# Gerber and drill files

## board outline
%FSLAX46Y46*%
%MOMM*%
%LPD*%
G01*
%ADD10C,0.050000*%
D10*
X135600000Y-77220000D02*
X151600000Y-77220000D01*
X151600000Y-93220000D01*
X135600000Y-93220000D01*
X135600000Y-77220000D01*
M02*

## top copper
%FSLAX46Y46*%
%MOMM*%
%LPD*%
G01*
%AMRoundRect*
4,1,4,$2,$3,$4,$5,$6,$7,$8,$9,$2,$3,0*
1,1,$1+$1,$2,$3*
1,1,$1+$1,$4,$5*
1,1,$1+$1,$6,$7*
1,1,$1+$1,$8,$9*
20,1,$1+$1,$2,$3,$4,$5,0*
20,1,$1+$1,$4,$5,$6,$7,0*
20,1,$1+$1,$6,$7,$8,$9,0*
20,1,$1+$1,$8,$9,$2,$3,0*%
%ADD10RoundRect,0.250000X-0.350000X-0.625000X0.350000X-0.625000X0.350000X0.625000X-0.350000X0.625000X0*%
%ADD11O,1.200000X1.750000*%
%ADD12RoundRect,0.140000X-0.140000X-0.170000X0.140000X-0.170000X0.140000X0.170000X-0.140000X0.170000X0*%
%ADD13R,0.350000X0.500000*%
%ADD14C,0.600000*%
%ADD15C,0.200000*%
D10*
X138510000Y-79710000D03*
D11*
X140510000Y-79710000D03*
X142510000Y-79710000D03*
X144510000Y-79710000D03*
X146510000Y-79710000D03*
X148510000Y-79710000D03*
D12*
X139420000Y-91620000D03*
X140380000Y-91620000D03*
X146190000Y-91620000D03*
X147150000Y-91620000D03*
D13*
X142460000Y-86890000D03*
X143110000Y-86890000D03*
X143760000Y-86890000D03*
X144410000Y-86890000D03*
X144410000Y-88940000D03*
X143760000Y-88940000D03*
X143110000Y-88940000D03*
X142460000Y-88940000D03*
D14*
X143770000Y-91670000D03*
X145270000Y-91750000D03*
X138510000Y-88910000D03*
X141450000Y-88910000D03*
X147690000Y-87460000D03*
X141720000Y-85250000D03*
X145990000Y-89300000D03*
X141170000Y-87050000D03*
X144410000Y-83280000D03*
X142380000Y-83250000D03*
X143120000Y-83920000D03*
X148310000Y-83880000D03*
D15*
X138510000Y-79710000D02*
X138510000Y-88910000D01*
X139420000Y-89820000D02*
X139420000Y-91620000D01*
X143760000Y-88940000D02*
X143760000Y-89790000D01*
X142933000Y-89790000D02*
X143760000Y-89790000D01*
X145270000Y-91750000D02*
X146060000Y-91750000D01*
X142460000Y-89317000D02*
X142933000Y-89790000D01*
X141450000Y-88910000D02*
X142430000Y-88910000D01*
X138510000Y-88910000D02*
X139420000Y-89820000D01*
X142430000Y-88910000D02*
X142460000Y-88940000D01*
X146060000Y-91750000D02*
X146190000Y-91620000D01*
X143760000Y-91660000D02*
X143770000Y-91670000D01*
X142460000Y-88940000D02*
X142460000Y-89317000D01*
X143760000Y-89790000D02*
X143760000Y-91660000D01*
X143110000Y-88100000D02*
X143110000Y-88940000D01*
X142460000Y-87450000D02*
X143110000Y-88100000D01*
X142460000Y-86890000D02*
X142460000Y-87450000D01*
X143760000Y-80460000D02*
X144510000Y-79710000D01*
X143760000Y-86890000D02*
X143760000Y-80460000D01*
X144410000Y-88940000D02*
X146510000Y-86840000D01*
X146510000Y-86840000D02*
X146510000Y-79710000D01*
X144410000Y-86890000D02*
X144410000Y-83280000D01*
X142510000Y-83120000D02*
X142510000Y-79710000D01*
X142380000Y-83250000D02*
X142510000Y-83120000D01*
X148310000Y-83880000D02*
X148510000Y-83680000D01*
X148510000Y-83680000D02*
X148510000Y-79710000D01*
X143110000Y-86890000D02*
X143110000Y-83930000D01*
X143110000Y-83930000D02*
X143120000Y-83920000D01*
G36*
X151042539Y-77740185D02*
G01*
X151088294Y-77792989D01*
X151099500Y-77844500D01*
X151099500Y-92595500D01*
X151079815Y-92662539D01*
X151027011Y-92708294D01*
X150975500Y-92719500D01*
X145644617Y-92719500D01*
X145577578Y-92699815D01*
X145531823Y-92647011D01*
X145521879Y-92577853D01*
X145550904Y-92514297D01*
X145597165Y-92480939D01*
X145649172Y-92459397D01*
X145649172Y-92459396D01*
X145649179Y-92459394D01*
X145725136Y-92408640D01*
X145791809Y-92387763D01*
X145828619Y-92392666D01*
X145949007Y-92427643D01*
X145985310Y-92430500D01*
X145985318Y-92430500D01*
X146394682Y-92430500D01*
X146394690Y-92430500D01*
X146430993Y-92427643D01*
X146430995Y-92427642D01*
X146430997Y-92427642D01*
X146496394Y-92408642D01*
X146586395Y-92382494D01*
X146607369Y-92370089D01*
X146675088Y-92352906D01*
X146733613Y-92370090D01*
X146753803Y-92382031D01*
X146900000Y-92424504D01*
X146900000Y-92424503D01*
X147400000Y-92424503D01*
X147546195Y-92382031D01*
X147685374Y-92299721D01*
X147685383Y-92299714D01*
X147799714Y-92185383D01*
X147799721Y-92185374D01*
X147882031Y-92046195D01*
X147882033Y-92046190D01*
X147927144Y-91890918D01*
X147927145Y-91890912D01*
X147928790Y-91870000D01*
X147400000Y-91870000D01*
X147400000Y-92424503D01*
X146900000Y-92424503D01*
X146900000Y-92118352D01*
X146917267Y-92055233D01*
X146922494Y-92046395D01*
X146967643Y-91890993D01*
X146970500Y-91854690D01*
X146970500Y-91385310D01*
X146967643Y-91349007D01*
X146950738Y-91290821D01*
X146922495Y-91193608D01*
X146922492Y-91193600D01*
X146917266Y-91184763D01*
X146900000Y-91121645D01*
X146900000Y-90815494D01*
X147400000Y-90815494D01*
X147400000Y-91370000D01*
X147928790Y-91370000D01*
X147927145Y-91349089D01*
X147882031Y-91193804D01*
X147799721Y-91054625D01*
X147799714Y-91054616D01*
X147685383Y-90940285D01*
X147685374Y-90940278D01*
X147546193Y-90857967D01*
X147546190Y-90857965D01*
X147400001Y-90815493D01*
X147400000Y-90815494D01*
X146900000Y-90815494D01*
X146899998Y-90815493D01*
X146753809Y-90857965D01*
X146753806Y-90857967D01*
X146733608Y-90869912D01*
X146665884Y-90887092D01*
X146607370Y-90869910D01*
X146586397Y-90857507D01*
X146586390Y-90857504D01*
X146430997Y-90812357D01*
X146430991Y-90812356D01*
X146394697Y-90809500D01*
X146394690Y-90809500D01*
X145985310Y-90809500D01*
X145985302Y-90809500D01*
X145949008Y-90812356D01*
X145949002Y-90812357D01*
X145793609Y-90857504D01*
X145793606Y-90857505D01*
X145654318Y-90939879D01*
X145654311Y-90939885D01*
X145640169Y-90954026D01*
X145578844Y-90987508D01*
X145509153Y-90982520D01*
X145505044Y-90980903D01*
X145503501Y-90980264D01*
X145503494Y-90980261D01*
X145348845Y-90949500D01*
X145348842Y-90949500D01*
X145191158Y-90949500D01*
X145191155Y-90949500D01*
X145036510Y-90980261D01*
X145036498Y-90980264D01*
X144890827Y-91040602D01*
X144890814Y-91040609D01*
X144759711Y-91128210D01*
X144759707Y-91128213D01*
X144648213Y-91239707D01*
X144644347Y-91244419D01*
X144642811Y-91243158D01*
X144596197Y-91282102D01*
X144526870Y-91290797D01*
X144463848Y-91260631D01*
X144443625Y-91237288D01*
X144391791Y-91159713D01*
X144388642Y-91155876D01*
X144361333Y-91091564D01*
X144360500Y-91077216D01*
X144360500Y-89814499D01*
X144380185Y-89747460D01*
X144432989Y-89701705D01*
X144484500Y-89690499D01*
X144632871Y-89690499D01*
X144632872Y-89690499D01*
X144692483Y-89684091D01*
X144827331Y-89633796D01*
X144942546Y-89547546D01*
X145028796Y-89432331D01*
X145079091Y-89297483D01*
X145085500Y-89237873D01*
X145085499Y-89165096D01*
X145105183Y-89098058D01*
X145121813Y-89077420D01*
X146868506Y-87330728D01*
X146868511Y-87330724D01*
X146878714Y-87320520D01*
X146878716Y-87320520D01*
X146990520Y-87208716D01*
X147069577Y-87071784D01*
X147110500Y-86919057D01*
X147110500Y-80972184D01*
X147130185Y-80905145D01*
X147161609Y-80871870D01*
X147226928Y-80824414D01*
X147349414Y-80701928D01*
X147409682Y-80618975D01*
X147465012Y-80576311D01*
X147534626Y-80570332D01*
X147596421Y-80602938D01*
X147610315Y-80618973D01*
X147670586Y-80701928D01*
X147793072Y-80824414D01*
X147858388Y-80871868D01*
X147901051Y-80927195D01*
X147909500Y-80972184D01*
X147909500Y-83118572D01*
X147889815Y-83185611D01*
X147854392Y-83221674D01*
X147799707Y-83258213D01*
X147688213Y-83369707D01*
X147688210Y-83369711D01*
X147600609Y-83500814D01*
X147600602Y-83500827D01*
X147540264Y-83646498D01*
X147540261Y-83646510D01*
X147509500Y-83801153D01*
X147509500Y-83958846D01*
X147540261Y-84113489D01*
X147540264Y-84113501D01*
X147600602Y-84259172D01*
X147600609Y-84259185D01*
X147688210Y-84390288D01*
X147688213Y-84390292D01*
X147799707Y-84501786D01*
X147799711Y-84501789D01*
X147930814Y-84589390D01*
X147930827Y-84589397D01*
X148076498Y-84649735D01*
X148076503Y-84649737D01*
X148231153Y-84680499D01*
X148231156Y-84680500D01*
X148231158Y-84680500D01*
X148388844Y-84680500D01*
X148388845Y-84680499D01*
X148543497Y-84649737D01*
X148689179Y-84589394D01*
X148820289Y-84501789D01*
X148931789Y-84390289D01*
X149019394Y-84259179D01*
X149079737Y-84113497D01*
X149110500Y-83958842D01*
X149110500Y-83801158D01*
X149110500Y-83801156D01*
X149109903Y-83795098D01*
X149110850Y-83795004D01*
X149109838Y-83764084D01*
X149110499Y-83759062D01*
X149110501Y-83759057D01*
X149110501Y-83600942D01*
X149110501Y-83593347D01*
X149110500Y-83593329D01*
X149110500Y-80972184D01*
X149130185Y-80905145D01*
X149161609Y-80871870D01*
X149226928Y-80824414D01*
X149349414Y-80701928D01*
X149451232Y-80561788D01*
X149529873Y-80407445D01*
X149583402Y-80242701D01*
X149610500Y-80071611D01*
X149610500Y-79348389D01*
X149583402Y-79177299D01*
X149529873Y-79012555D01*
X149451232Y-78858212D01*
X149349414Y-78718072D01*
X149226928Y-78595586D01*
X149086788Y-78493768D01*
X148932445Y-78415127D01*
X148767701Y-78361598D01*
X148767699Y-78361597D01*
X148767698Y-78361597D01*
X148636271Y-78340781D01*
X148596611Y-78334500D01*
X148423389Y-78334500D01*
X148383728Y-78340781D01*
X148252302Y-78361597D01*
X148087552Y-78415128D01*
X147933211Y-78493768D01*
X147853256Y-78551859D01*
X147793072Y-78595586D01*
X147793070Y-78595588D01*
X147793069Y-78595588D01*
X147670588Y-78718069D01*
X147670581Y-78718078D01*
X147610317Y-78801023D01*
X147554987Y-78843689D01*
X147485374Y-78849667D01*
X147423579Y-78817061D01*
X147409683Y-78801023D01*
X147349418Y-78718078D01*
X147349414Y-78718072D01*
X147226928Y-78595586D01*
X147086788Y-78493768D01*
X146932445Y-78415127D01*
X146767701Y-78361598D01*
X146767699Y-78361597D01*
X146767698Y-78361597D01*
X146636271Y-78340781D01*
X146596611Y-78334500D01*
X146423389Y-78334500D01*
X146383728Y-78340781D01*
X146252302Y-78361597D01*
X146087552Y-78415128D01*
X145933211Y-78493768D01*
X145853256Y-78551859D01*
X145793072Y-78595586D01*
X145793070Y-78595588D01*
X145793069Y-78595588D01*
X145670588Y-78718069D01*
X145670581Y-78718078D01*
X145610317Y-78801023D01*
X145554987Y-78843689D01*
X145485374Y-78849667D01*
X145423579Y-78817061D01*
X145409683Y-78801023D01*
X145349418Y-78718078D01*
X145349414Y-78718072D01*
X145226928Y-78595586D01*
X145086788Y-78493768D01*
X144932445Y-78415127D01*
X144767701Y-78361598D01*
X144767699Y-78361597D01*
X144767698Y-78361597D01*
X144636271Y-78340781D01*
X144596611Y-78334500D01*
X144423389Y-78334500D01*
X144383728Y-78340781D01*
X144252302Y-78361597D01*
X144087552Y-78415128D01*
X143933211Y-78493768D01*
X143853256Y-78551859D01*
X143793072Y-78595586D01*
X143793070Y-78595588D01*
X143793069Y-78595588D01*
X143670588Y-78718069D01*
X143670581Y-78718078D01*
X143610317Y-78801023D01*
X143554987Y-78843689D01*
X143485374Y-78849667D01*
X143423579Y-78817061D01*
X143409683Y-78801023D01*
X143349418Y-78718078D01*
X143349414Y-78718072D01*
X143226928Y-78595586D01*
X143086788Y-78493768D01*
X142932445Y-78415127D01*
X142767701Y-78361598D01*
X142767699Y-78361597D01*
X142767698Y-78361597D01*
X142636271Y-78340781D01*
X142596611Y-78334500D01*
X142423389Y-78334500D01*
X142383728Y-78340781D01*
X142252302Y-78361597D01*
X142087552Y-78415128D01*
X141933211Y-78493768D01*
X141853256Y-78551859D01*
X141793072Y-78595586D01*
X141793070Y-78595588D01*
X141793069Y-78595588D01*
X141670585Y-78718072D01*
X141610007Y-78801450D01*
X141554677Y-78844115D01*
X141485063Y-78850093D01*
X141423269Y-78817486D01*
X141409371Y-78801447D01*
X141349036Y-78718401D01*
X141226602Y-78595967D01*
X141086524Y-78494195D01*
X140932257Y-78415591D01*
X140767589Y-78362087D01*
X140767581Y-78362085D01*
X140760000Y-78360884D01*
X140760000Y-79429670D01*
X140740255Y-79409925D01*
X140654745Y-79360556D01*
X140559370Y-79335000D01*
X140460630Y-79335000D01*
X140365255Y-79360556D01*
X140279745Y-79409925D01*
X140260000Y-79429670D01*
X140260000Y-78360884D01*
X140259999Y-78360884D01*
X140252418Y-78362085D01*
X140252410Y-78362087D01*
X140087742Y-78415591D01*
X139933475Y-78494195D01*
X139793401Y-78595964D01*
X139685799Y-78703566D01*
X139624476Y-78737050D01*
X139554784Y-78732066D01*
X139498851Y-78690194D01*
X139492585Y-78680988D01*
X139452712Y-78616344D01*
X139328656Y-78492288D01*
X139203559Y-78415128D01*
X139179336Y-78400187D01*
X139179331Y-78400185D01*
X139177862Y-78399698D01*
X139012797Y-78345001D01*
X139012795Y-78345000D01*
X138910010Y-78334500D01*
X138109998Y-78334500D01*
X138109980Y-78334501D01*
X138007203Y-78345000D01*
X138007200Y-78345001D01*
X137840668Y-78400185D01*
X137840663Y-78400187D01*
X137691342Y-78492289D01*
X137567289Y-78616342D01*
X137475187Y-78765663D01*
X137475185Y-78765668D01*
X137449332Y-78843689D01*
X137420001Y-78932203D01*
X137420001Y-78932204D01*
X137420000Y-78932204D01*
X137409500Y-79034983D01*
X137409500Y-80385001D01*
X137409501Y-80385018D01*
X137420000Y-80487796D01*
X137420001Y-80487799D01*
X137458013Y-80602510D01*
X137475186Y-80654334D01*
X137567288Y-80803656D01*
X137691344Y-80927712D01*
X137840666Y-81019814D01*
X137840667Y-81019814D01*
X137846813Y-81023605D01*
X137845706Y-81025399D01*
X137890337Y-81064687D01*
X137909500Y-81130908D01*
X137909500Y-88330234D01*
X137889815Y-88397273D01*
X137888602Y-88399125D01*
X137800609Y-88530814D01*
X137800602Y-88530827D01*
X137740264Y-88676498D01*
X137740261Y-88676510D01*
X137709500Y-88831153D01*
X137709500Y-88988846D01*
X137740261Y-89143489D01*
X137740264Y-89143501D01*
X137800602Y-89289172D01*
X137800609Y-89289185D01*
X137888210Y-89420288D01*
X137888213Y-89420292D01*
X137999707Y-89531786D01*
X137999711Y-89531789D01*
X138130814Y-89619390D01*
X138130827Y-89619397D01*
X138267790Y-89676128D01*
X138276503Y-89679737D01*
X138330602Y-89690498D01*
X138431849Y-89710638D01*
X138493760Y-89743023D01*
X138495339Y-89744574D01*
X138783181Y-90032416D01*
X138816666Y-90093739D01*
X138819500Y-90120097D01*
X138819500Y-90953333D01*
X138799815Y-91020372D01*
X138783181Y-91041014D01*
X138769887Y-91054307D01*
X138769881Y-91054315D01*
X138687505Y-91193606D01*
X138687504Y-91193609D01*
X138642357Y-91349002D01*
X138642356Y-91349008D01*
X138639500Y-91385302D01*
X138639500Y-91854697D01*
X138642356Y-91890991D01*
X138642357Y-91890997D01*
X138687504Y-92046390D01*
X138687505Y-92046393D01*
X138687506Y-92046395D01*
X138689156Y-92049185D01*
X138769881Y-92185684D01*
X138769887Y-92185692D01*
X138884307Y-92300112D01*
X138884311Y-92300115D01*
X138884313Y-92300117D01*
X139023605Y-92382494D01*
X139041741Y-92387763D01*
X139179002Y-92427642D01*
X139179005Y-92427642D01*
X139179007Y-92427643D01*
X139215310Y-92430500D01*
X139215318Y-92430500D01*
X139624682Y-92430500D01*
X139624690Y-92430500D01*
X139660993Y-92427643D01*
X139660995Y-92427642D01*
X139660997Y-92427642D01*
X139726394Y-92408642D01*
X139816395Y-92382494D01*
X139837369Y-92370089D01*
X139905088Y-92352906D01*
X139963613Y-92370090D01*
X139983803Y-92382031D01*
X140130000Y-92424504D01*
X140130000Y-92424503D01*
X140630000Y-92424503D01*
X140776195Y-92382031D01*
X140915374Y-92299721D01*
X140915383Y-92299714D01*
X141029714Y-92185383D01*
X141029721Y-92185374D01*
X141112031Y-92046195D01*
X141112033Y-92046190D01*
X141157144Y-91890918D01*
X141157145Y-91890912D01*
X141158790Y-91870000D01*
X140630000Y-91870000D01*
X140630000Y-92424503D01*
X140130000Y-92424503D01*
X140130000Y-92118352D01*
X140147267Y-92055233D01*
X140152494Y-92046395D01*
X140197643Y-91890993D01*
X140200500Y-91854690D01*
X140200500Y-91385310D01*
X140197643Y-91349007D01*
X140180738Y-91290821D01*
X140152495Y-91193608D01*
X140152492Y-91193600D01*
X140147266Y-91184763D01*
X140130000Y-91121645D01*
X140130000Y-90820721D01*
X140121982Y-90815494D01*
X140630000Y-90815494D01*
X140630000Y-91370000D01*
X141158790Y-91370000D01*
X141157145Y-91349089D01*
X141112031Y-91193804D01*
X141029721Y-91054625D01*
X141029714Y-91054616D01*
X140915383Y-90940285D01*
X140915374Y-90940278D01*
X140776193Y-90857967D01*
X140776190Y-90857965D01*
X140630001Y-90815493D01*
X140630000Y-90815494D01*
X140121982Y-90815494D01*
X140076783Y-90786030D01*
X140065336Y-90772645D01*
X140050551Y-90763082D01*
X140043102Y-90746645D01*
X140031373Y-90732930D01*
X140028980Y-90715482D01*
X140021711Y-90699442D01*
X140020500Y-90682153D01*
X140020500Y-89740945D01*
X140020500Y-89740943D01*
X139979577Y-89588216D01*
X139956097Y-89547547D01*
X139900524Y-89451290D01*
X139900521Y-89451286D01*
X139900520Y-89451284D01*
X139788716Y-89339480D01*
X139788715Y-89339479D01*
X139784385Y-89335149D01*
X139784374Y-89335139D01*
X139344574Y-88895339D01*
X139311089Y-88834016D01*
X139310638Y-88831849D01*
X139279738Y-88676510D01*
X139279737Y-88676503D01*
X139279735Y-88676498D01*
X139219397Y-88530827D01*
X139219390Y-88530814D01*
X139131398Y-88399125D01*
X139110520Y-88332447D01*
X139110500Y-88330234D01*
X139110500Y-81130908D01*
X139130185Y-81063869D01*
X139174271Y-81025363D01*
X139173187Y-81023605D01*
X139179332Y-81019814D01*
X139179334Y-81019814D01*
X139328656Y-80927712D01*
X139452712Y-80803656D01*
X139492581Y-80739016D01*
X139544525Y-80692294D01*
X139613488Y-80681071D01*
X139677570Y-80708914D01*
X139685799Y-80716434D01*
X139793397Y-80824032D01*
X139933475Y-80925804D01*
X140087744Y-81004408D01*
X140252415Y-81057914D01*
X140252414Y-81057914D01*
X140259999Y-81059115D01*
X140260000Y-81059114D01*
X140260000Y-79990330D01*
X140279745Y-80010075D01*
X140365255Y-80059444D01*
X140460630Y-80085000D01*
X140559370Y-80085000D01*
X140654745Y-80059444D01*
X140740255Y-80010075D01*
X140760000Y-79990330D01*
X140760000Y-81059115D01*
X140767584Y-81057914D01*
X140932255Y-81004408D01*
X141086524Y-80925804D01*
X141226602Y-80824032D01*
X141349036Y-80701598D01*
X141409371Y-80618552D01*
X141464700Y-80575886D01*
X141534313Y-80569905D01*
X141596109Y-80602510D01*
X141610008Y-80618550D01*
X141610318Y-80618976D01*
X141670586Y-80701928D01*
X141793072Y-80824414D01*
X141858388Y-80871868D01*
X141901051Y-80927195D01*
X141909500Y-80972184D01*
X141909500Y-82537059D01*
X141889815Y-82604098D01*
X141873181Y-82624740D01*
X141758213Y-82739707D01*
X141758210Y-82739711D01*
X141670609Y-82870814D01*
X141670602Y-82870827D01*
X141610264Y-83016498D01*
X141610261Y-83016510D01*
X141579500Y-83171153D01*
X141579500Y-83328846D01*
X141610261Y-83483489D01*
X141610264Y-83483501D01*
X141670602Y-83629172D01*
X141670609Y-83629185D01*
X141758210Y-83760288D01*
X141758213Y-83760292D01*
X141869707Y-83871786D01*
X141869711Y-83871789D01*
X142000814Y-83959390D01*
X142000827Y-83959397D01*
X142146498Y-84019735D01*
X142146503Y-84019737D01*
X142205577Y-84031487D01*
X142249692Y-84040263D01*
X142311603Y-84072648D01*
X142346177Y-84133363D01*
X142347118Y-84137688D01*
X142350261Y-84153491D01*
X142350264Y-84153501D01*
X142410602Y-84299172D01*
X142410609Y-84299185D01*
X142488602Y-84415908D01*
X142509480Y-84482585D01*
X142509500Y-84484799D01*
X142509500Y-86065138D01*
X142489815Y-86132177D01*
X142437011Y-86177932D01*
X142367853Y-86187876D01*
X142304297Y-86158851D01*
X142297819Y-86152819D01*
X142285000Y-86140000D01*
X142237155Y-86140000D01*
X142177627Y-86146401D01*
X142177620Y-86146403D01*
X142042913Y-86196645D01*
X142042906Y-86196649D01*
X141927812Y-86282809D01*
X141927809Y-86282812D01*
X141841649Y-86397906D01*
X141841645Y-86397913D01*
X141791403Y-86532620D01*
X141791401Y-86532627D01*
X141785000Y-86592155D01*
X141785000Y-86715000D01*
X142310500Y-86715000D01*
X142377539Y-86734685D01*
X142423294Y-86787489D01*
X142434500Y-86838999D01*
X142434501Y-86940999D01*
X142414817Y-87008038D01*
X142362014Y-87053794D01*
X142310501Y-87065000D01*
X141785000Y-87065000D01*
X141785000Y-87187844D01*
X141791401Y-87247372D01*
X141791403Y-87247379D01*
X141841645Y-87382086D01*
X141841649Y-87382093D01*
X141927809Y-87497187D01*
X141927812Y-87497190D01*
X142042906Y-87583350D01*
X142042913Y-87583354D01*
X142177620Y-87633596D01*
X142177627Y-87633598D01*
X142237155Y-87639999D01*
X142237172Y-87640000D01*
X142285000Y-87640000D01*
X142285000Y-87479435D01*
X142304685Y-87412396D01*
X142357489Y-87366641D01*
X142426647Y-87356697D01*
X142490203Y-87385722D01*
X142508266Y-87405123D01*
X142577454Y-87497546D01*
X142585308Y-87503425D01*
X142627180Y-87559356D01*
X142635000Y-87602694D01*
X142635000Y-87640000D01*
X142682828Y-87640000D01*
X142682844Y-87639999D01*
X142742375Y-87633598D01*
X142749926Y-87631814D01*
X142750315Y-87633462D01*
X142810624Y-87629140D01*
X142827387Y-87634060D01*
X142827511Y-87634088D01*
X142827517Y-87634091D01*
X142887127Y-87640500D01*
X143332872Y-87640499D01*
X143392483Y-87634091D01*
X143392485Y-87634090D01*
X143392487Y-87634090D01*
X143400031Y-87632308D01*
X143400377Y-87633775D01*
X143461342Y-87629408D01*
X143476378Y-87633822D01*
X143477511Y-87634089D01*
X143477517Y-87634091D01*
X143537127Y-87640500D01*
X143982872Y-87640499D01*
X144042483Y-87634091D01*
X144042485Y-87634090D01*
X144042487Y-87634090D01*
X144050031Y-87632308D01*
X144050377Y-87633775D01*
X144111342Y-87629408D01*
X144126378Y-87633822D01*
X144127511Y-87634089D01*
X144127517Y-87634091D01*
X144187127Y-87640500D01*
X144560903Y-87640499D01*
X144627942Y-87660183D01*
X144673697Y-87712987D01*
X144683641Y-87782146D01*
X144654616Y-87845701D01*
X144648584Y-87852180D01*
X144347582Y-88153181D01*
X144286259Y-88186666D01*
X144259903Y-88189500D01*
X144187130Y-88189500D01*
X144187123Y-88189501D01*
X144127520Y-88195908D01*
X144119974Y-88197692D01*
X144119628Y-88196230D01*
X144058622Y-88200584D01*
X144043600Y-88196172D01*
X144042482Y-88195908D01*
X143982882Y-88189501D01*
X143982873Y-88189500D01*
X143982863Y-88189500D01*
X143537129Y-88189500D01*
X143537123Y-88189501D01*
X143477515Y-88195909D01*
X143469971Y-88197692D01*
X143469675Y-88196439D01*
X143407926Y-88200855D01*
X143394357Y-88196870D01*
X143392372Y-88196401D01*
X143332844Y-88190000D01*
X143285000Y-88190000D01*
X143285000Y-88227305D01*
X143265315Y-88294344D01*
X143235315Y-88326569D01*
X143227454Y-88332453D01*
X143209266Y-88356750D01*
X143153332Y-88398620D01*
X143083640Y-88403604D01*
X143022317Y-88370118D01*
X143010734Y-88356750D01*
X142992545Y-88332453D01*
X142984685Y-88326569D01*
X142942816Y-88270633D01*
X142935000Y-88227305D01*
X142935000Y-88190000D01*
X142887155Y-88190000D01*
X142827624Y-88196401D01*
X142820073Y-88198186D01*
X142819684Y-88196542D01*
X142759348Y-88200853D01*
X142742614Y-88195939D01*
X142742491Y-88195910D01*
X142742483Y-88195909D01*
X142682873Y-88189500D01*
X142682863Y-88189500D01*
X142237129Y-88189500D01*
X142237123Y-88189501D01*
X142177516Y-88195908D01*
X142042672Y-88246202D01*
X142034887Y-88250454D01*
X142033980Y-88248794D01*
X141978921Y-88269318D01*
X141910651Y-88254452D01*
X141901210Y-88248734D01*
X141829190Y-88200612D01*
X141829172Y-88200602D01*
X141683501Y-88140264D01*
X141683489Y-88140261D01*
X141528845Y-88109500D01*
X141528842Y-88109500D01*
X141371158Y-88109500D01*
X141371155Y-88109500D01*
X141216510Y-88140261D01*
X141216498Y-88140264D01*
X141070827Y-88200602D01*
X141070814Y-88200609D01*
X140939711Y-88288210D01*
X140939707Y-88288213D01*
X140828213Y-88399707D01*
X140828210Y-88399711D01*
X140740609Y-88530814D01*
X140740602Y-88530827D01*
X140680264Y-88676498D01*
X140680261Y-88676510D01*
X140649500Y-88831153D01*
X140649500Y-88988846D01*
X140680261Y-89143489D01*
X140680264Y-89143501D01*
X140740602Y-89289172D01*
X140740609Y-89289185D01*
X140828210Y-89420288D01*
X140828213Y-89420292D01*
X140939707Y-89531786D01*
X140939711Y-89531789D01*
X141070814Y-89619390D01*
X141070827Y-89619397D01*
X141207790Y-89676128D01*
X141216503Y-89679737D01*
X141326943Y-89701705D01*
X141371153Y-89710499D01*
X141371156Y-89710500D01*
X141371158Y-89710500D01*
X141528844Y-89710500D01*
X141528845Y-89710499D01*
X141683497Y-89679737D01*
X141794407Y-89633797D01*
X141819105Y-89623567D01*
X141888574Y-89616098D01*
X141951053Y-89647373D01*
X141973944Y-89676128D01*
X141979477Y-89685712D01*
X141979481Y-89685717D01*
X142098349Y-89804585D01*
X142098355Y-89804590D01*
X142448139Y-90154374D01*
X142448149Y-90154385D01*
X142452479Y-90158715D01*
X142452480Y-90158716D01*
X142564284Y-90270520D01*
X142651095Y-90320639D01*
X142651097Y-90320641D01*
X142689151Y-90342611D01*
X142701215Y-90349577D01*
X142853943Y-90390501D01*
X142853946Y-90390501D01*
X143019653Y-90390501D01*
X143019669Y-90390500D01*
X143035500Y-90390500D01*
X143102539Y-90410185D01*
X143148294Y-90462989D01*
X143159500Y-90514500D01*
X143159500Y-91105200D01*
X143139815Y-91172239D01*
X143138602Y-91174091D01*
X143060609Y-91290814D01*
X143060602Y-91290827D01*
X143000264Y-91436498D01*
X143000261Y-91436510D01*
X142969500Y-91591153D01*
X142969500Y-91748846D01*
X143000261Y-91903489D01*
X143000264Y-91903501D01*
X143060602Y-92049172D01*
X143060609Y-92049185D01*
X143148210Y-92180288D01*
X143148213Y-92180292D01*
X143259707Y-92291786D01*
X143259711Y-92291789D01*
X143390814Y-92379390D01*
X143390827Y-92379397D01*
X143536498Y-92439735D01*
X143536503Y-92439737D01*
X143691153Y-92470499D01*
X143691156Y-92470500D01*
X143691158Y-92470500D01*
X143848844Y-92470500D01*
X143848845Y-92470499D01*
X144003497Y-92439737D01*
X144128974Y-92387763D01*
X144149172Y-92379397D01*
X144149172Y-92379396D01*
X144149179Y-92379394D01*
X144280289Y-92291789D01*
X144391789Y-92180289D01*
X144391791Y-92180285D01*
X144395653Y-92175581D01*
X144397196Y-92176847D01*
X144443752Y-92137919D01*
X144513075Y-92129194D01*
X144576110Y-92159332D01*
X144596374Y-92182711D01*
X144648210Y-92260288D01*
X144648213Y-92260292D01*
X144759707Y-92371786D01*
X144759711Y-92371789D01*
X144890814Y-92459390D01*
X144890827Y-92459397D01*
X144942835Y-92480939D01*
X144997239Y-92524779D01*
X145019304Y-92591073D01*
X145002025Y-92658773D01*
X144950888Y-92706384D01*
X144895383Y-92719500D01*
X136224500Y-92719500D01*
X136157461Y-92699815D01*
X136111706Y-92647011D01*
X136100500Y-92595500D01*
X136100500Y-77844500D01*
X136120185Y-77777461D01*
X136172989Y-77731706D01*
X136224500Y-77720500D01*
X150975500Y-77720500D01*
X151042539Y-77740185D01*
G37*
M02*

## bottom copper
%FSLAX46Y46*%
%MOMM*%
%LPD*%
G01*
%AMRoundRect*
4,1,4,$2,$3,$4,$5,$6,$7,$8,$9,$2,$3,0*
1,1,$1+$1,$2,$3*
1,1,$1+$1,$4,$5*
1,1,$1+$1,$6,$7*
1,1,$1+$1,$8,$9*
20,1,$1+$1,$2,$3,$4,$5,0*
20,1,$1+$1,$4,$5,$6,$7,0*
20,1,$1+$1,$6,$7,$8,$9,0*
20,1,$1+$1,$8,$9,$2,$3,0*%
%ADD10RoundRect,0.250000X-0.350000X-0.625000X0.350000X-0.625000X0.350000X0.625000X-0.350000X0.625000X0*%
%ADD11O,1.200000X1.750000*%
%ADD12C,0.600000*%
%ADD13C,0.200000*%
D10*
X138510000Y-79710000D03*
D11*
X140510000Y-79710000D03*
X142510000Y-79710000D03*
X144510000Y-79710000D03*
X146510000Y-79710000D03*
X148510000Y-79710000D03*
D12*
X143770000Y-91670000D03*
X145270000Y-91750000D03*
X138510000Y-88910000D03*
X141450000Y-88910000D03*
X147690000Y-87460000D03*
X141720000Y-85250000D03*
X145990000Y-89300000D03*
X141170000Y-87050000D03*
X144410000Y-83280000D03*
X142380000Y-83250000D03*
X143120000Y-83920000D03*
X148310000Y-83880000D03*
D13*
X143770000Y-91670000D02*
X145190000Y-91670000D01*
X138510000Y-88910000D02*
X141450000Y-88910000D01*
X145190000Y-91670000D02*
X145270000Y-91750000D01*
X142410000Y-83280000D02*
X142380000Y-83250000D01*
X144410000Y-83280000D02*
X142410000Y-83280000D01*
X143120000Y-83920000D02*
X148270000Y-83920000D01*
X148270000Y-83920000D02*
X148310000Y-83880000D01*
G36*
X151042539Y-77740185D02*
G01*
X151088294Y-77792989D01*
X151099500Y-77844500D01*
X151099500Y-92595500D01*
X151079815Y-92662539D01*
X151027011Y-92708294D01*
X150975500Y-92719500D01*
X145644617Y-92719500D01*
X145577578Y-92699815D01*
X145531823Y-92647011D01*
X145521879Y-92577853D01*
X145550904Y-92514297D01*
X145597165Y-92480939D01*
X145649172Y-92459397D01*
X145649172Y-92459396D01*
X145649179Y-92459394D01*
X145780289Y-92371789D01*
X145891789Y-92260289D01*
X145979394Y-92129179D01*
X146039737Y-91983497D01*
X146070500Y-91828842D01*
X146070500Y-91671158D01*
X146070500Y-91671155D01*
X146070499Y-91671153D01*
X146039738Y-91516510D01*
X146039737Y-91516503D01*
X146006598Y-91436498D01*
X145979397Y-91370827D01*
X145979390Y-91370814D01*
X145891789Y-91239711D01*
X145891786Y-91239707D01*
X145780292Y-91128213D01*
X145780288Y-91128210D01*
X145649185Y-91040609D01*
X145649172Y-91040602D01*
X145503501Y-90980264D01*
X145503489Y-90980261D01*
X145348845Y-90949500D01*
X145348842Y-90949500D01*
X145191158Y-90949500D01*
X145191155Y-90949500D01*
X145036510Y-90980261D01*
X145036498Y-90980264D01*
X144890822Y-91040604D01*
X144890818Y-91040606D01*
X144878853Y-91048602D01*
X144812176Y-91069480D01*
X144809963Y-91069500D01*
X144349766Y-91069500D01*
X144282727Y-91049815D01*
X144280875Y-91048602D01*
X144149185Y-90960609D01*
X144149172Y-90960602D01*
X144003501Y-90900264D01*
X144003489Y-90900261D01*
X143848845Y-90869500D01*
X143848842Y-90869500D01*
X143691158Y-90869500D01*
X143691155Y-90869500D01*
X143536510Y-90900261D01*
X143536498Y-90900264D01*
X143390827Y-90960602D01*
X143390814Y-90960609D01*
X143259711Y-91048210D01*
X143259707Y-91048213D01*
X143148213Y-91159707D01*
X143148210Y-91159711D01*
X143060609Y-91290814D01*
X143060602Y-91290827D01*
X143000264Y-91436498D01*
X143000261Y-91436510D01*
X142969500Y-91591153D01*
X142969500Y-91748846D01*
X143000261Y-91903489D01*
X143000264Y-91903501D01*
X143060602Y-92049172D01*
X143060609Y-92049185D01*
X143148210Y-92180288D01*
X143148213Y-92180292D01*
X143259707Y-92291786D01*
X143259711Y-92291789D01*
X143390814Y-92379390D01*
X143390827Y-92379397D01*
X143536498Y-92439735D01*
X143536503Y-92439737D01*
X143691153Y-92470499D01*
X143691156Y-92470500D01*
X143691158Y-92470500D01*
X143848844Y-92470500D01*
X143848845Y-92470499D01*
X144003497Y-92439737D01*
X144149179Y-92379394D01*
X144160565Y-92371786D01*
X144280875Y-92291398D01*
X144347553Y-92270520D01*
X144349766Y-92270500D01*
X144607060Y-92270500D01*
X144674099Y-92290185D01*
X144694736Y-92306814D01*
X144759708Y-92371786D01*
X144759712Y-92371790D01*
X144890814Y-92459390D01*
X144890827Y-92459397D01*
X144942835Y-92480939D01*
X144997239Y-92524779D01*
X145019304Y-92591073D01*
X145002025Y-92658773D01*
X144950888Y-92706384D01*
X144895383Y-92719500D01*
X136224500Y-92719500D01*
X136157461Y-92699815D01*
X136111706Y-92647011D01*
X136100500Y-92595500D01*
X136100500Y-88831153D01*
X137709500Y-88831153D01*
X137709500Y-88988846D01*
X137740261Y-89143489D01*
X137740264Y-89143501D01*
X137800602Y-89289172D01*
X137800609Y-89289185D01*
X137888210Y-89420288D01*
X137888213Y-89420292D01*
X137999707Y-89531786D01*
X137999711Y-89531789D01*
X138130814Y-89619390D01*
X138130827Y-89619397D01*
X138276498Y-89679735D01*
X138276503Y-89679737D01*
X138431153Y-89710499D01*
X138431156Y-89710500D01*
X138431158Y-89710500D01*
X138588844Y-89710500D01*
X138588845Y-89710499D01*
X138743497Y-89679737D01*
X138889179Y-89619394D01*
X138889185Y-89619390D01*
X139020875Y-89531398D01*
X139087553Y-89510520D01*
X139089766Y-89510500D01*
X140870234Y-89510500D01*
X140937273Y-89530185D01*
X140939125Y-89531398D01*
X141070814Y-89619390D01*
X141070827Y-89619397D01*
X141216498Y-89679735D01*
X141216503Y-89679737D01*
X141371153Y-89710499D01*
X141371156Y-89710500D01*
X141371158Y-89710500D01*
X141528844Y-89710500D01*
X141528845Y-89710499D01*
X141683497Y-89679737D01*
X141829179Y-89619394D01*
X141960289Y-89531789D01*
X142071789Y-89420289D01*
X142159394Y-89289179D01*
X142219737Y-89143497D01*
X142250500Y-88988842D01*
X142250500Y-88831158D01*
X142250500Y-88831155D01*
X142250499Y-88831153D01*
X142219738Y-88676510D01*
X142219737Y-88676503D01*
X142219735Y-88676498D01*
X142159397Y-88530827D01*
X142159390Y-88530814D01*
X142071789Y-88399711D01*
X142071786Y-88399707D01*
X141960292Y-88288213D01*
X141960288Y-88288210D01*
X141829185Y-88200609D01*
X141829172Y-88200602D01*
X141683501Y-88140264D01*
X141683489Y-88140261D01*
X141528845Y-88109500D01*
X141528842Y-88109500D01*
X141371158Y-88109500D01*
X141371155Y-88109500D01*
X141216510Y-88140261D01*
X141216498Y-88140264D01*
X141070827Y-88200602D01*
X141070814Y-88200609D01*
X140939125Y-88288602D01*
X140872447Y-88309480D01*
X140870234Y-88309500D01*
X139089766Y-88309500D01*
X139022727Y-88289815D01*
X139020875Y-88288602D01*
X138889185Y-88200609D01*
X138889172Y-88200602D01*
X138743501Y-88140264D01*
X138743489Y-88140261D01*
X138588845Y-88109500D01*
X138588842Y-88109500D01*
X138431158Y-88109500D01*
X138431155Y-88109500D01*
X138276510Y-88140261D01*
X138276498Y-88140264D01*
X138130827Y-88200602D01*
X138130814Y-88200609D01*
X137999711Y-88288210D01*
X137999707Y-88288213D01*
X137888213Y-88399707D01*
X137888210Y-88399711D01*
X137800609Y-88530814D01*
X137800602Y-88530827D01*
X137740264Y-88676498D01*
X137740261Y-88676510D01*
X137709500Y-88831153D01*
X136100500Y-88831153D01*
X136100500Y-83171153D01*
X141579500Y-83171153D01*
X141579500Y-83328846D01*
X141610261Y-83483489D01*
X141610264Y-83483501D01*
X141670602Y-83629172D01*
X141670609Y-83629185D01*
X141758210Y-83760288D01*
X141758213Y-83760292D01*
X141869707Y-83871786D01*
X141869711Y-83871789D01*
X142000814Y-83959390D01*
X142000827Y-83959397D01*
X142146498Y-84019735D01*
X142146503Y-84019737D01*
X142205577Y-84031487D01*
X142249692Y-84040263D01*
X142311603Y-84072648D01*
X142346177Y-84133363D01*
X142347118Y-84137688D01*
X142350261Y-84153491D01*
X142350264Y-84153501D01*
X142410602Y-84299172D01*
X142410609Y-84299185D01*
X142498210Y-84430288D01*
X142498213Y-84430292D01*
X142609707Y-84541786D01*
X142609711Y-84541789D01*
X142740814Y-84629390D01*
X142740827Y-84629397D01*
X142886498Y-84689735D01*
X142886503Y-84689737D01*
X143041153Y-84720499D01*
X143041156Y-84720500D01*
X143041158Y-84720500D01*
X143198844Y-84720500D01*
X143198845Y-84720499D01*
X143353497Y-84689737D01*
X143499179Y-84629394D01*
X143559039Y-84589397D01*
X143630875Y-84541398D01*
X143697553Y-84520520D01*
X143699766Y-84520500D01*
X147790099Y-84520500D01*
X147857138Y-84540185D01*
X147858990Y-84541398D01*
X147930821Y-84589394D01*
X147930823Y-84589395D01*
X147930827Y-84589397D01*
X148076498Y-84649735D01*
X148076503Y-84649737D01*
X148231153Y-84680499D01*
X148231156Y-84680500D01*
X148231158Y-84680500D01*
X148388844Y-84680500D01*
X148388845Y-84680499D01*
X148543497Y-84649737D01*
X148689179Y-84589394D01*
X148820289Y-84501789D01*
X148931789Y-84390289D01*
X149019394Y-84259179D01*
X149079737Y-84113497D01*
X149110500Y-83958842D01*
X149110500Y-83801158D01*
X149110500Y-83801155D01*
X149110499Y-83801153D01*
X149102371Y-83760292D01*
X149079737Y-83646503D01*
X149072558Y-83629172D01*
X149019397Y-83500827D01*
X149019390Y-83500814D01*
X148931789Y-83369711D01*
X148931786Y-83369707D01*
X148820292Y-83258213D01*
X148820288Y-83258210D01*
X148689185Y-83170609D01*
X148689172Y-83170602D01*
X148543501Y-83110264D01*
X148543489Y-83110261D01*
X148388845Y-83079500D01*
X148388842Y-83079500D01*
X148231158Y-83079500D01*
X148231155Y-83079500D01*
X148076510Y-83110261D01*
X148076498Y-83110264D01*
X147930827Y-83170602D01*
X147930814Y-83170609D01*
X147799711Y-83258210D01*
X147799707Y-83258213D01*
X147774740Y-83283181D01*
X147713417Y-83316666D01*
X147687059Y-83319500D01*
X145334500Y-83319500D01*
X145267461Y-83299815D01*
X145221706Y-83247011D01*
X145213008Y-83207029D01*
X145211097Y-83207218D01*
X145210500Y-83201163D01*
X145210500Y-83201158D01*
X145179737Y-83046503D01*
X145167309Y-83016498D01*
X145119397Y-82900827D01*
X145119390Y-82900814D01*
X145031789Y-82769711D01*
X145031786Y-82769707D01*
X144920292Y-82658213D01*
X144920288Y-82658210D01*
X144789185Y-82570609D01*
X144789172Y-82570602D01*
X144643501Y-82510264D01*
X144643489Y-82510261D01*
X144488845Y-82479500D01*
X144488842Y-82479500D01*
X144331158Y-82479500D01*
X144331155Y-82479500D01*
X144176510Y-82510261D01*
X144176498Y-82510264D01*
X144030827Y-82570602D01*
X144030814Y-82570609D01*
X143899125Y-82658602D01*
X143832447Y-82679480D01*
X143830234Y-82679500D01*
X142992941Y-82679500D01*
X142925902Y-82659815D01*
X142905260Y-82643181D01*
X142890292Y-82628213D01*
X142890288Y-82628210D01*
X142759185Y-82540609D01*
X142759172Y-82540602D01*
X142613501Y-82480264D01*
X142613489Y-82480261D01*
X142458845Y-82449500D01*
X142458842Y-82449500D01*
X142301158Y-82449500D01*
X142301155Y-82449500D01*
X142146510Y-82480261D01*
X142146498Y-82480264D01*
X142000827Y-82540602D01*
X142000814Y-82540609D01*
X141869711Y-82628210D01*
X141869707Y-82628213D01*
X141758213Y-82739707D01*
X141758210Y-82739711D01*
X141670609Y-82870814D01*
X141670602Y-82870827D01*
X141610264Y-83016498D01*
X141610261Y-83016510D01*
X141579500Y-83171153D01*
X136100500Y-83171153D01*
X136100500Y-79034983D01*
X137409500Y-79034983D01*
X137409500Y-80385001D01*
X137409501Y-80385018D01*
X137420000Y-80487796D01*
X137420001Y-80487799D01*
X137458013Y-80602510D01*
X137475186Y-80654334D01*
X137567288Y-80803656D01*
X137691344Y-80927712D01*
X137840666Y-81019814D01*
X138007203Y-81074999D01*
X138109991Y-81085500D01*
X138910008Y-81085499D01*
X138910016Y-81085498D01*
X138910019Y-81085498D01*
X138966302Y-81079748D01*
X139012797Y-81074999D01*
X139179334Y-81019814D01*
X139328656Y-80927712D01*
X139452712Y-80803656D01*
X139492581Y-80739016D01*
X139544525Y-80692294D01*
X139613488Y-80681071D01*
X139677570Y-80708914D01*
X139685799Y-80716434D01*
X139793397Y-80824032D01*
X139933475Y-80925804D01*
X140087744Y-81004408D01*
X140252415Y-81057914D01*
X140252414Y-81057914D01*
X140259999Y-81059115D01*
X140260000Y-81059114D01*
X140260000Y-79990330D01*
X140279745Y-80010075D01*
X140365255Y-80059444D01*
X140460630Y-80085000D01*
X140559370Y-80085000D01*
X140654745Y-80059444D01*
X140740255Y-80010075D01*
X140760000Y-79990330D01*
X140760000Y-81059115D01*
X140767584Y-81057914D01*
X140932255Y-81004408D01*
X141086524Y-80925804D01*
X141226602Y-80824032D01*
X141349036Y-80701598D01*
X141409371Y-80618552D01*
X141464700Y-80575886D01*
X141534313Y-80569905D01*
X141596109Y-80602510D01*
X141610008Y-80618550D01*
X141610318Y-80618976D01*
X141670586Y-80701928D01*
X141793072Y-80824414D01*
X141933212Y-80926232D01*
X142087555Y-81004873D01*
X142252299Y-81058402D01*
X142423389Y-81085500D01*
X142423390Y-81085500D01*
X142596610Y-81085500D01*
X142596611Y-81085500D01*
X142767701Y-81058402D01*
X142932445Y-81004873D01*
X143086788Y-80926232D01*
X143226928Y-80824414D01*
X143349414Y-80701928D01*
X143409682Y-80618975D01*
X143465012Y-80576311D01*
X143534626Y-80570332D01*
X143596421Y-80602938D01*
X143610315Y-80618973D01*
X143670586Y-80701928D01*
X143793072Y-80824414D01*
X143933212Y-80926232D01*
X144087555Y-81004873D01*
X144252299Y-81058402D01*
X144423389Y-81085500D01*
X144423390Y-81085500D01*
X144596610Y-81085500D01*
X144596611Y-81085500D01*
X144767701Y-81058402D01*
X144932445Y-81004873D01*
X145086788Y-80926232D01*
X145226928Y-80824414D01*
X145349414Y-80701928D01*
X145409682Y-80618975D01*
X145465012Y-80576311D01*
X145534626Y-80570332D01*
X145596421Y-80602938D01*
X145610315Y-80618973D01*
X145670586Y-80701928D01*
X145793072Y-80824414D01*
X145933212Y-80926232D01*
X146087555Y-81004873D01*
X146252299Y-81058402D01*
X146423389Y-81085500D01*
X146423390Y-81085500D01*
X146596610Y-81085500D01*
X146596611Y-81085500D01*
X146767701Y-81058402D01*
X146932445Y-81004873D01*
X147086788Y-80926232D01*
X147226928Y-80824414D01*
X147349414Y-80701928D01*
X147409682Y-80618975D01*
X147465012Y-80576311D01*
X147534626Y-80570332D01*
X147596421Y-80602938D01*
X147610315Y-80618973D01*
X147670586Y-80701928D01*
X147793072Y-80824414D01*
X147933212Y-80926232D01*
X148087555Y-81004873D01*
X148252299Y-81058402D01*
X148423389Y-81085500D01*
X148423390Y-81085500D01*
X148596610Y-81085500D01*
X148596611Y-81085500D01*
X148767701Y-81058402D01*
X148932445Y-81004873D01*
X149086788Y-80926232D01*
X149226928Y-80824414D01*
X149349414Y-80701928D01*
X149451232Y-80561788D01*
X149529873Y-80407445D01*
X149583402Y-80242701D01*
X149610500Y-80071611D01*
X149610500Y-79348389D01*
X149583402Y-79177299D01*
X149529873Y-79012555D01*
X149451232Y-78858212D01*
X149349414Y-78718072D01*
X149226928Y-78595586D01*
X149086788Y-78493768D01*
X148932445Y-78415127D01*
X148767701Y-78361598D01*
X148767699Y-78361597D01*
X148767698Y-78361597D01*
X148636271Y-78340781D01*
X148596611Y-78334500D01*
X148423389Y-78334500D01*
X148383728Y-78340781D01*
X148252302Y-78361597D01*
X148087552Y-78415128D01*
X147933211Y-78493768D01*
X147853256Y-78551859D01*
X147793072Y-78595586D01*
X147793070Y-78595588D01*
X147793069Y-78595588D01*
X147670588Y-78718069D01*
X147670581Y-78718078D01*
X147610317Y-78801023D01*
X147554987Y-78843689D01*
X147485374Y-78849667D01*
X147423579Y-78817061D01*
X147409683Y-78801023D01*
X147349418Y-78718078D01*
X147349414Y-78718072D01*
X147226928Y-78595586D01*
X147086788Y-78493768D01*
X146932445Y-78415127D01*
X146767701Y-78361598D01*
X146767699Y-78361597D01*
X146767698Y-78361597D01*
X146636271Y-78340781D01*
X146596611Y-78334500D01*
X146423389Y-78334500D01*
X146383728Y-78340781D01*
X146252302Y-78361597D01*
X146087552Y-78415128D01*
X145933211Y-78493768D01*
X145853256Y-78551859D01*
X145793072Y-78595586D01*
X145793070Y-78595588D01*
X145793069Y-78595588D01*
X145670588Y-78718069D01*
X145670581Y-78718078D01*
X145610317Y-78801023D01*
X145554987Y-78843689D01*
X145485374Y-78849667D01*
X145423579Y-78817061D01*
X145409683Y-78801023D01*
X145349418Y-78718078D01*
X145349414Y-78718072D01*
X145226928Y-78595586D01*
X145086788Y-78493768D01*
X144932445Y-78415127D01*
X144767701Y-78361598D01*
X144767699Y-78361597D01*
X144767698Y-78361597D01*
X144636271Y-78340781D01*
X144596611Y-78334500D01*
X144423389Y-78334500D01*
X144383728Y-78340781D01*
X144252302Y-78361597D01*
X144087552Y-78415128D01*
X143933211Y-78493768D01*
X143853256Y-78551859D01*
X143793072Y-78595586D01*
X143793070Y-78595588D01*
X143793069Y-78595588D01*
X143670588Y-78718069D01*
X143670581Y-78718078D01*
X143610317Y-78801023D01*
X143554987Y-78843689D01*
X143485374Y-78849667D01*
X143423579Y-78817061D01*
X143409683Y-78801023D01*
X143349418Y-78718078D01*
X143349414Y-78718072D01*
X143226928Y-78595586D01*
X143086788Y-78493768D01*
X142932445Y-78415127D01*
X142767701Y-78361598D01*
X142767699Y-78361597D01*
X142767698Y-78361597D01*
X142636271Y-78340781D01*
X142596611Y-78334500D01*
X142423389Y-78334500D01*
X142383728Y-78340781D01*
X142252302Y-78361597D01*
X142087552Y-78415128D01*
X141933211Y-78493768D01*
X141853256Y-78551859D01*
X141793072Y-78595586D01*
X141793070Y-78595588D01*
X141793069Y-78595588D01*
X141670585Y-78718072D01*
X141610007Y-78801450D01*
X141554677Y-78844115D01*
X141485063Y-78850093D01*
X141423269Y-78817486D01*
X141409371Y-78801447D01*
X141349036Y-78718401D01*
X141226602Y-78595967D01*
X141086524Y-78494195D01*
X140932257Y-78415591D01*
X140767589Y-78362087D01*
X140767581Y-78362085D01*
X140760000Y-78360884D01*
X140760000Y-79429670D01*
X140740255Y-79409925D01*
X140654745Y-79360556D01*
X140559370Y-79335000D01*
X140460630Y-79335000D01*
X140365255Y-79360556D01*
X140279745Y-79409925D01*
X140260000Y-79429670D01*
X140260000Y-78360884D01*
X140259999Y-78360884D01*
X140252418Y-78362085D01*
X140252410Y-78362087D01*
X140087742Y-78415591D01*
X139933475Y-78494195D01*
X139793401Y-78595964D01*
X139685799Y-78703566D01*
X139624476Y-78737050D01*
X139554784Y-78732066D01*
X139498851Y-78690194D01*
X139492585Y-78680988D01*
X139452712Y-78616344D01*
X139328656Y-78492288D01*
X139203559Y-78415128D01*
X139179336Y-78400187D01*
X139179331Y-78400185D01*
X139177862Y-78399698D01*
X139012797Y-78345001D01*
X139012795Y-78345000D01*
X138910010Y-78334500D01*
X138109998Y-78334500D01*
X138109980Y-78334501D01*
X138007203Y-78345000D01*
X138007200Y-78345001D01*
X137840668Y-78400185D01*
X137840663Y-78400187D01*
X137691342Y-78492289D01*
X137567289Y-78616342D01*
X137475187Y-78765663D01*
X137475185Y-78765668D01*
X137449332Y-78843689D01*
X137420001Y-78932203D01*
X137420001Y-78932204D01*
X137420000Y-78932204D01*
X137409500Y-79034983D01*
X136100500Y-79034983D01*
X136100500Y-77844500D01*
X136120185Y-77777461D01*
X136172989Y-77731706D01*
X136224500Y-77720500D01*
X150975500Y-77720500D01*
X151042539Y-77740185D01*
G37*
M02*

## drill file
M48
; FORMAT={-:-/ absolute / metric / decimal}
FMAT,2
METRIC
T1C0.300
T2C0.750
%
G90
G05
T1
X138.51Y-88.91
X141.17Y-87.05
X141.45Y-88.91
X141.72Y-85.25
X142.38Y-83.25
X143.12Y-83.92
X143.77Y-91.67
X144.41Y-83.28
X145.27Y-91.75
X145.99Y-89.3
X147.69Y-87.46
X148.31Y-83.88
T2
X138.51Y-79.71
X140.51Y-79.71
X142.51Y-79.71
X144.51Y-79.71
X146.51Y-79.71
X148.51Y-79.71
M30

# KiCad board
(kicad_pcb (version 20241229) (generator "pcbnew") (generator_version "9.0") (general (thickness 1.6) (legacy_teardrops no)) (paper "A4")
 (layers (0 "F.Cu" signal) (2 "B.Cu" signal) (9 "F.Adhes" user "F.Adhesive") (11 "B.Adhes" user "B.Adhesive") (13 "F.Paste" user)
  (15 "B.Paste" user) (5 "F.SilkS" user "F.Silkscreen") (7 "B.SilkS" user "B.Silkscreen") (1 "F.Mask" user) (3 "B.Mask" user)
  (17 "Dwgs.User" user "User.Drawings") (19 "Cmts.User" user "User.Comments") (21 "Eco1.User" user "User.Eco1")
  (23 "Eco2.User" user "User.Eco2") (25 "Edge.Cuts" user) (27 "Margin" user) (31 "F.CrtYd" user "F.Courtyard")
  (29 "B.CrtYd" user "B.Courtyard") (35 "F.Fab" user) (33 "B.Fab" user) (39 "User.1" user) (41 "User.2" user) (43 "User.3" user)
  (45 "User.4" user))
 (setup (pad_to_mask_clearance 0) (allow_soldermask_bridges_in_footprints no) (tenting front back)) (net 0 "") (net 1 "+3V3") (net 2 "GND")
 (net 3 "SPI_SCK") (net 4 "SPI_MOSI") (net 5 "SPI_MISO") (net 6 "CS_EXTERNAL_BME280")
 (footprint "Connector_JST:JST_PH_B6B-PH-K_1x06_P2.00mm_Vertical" (layer "F.Cu") (at 138.51 79.71)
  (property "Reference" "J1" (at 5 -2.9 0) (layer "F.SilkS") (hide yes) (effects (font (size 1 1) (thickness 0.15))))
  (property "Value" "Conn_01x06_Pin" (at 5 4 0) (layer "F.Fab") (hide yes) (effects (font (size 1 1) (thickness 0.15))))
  (pad "1" thru_hole roundrect (at 0 0) (size 1.2 1.75) (drill 0.75) (layers "*.Cu" "*.Mask") (remove_unused_layers no)
   (roundrect_rratio 0.208333) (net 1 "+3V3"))
  (pad "2" thru_hole oval (at 2 0) (size 1.2 1.75) (drill 0.75) (layers "*.Cu" "*.Mask") (remove_unused_layers no) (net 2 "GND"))
  (pad "3" thru_hole oval (at 4 0) (size 1.2 1.75) (drill 0.75) (layers "*.Cu" "*.Mask") (remove_unused_layers no) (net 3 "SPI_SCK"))
  (pad "4" thru_hole oval (at 6 0) (size 1.2 1.75) (drill 0.75) (layers "*.Cu" "*.Mask") (remove_unused_layers no) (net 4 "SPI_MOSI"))
  (pad "5" thru_hole oval (at 8 0) (size 1.2 1.75) (drill 0.75) (layers "*.Cu" "*.Mask") (remove_unused_layers no) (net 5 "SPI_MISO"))
  (pad "6" thru_hole oval (at 10 0) (size 1.2 1.75) (drill 0.75) (layers "*.Cu" "*.Mask") (remove_unused_layers no)
   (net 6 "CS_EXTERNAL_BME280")))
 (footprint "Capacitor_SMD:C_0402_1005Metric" (layer "F.Cu") (at 139.9 91.62)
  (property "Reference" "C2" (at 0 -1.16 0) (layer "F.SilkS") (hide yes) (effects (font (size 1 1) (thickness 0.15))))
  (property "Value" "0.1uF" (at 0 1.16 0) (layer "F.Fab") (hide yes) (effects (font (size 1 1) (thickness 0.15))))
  (pad "1" smd roundrect (at -0.48 0) (size 0.56 0.62) (layers "F.Cu" "F.Mask" "F.Paste") (roundrect_rratio 0.25) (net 1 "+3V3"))
  (pad "2" smd roundrect (at 0.48 0) (size 0.56 0.62) (layers "F.Cu" "F.Mask" "F.Paste") (roundrect_rratio 0.25) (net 2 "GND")))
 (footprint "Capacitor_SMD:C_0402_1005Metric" (layer "F.Cu") (at 146.67 91.62)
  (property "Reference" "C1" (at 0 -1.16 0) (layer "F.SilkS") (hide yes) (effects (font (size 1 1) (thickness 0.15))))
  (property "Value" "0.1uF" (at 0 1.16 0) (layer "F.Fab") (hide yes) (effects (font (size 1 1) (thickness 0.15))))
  (pad "1" smd roundrect (at -0.48 0) (size 0.56 0.62) (layers "F.Cu" "F.Mask" "F.Paste") (roundrect_rratio 0.25) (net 1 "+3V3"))
  (pad "2" smd roundrect (at 0.48 0) (size 0.56 0.62) (layers "F.Cu" "F.Mask" "F.Paste") (roundrect_rratio 0.25) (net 2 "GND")))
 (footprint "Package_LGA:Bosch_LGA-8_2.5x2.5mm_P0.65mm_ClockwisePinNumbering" (layer "F.Cu") (at 143.435 87.915)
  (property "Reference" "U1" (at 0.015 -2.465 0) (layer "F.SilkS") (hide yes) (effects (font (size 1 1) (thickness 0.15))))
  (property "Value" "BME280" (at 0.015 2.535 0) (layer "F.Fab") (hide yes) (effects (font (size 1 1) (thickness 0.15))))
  (pad "1" smd rect (at -0.975 -1.025 90) (size 0.5 0.35) (layers "F.Cu" "F.Mask" "F.Paste") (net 2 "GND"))
  (pad "2" smd rect (at -0.325 -1.025 90) (size 0.5 0.35) (layers "F.Cu" "F.Mask" "F.Paste") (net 6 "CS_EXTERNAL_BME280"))
  (pad "3" smd rect (at 0.325 -1.025 90) (size 0.5 0.35) (layers "F.Cu" "F.Mask" "F.Paste") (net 4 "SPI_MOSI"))
  (pad "4" smd rect (at 0.975 -1.025 90) (size 0.5 0.35) (layers "F.Cu" "F.Mask" "F.Paste") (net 3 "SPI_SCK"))
  (pad "5" smd rect (at 0.975 1.025 90) (size 0.5 0.35) (layers "F.Cu" "F.Mask" "F.Paste") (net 5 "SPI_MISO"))
  (pad "6" smd rect (at 0.325 1.025 90) (size 0.5 0.35) (layers "F.Cu" "F.Mask" "F.Paste") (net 1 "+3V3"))
  (pad "7" smd rect (at -0.325 1.025 90) (size 0.5 0.35) (layers "F.Cu" "F.Mask" "F.Paste") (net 2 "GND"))
  (pad "8" smd rect (at -0.975 1.025 90) (size 0.5 0.35) (layers "F.Cu" "F.Mask" "F.Paste") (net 1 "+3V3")))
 (gr_rect (start 135.6 77.22) (end 151.6 93.22) (stroke (width 0.05) (type solid)) (fill no) (layer "Edge.Cuts"))
 (segment (start 138.51 79.71) (end 138.51 88.91) (width 0.2) (layer "F.Cu") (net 1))
 (segment (start 139.42 89.82) (end 139.42 91.62) (width 0.2) (layer "F.Cu") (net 1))
 (segment (start 143.76 88.94) (end 143.76 89.79) (width 0.2) (layer "F.Cu") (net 1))
 (segment (start 142.933 89.79) (end 143.76 89.79) (width 0.2) (layer "F.Cu") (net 1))
 (segment (start 145.27 91.75) (end 146.06 91.75) (width 0.2) (layer "F.Cu") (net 1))
 (segment (start 142.46 89.317) (end 142.933 89.79) (width 0.2) (layer "F.Cu") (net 1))
 (segment (start 141.45 88.91) (end 142.43 88.91) (width 0.2) (layer "F.Cu") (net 1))
 (segment (start 138.51 88.91) (end 139.42 89.82) (width 0.2) (layer "F.Cu") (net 1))
 (segment (start 142.43 88.91) (end 142.46 88.94) (width 0.2) (layer "F.Cu") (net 1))
 (segment (start 146.06 91.75) (end 146.19 91.62) (width 0.2) (layer "F.Cu") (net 1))
 (segment (start 143.76 91.66) (end 143.77 91.67) (width 0.2) (layer "F.Cu") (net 1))
 (segment (start 142.46 88.94) (end 142.46 89.317) (width 0.2) (layer "F.Cu") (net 1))
 (segment (start 143.76 89.79) (end 143.76 91.66) (width 0.2) (layer "F.Cu") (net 1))
 (via (at 143.77 91.67) (size 0.6) (drill 0.3) (layers "F.Cu" "B.Cu") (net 1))
 (via (at 145.27 91.75) (size 0.6) (drill 0.3) (layers "F.Cu" "B.Cu") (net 1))
 (via (at 138.51 88.91) (size 0.6) (drill 0.3) (layers "F.Cu" "B.Cu") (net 1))
 (via (at 141.45 88.91) (size 0.6) (drill 0.3) (layers "F.Cu" "B.Cu") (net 1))
 (segment (start 143.77 91.67) (end 145.19 91.67) (width 0.2) (layer "B.Cu") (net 1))
 (segment (start 138.51 88.91) (end 141.45 88.91) (width 0.2) (layer "B.Cu") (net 1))
 (segment (start 145.19 91.67) (end 145.27 91.75) (width 0.2) (layer "B.Cu") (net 1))
 (segment (start 143.11 88.1) (end 143.11 88.94) (width 0.2) (layer "F.Cu") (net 2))
 (segment (start 142.46 87.45) (end 143.11 88.1) (width 0.2) (layer "F.Cu") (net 2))
 (segment (start 142.46 86.89) (end 142.46 87.45) (width 0.2) (layer "F.Cu") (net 2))
 (via (at 147.69 87.46) (size 0.6) (drill 0.3) (layers "F.Cu" "B.Cu") (free yes) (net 2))
 (via (at 141.72 85.25) (size 0.6) (drill 0.3) (layers "F.Cu" "B.Cu") (free yes) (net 2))
 (via (at 145.99 89.3) (size 0.6) (drill 0.3) (layers "F.Cu" "B.Cu") (free yes) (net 2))
 (via (at 141.17 87.05) (size 0.6) (drill 0.3) (layers "F.Cu" "B.Cu") (free yes) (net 2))
 (segment (start 143.76 80.46) (end 144.51 79.71) (width 0.2) (layer "F.Cu") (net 4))
 (segment (start 143.76 86.89) (end 143.76 80.46) (width 0.2) (layer "F.Cu") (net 4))
 (segment (start 144.41 88.94) (end 146.51 86.84) (width 0.2) (layer "F.Cu") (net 5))
 (segment (start 146.51 86.84) (end 146.51 79.71) (width 0.2) (layer "F.Cu") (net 5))
 (segment (start 144.41 86.89) (end 144.41 83.28) (width 0.2) (layer "F.Cu") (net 3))
 (segment (start 142.51 83.12) (end 142.51 79.71) (width 0.2) (layer "F.Cu") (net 3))
 (segment (start 142.38 83.25) (end 142.51 83.12) (width 0.2) (layer "F.Cu") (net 3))
 (via (at 144.41 83.28) (size 0.6) (drill 0.3) (layers "F.Cu" "B.Cu") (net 3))
 (via (at 142.38 83.25) (size 0.6) (drill 0.3) (layers "F.Cu" "B.Cu") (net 3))
 (segment (start 142.41 83.28) (end 142.38 83.25) (width 0.2) (layer "B.Cu") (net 3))
 (segment (start 144.41 83.28) (end 142.41 83.28) (width 0.2) (layer "B.Cu") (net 3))
 (segment (start 148.31 83.88) (end 148.51 83.68) (width 0.2) (layer "F.Cu") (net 6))
 (segment (start 148.51 83.68) (end 148.51 79.71) (width 0.2) (layer "F.Cu") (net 6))
 (segment (start 143.11 86.89) (end 143.11 83.93) (width 0.2) (layer "F.Cu") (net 6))
 (segment (start 143.11 83.93) (end 143.12 83.92) (width 0.2) (layer "F.Cu") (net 6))
 (via (at 143.12 83.92) (size 0.6) (drill 0.3) (layers "F.Cu" "B.Cu") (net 6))
 (via (at 148.31 83.88) (size 0.6) (drill 0.3) (layers "F.Cu" "B.Cu") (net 6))
 (segment (start 143.12 83.92) (end 148.27 83.92) (width 0.2) (layer "B.Cu") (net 6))
 (segment (start 148.27 83.92) (end 148.31 83.88) (width 0.2) (layer "B.Cu") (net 6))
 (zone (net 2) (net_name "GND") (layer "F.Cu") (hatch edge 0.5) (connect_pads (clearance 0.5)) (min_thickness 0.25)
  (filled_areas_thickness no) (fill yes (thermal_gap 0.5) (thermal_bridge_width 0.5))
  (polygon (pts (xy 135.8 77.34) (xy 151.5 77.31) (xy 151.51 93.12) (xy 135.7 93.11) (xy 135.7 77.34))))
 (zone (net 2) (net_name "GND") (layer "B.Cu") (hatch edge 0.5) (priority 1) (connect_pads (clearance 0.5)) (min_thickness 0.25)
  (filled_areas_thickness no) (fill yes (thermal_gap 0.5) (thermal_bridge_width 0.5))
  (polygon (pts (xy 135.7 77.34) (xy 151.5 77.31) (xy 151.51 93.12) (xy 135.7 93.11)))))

